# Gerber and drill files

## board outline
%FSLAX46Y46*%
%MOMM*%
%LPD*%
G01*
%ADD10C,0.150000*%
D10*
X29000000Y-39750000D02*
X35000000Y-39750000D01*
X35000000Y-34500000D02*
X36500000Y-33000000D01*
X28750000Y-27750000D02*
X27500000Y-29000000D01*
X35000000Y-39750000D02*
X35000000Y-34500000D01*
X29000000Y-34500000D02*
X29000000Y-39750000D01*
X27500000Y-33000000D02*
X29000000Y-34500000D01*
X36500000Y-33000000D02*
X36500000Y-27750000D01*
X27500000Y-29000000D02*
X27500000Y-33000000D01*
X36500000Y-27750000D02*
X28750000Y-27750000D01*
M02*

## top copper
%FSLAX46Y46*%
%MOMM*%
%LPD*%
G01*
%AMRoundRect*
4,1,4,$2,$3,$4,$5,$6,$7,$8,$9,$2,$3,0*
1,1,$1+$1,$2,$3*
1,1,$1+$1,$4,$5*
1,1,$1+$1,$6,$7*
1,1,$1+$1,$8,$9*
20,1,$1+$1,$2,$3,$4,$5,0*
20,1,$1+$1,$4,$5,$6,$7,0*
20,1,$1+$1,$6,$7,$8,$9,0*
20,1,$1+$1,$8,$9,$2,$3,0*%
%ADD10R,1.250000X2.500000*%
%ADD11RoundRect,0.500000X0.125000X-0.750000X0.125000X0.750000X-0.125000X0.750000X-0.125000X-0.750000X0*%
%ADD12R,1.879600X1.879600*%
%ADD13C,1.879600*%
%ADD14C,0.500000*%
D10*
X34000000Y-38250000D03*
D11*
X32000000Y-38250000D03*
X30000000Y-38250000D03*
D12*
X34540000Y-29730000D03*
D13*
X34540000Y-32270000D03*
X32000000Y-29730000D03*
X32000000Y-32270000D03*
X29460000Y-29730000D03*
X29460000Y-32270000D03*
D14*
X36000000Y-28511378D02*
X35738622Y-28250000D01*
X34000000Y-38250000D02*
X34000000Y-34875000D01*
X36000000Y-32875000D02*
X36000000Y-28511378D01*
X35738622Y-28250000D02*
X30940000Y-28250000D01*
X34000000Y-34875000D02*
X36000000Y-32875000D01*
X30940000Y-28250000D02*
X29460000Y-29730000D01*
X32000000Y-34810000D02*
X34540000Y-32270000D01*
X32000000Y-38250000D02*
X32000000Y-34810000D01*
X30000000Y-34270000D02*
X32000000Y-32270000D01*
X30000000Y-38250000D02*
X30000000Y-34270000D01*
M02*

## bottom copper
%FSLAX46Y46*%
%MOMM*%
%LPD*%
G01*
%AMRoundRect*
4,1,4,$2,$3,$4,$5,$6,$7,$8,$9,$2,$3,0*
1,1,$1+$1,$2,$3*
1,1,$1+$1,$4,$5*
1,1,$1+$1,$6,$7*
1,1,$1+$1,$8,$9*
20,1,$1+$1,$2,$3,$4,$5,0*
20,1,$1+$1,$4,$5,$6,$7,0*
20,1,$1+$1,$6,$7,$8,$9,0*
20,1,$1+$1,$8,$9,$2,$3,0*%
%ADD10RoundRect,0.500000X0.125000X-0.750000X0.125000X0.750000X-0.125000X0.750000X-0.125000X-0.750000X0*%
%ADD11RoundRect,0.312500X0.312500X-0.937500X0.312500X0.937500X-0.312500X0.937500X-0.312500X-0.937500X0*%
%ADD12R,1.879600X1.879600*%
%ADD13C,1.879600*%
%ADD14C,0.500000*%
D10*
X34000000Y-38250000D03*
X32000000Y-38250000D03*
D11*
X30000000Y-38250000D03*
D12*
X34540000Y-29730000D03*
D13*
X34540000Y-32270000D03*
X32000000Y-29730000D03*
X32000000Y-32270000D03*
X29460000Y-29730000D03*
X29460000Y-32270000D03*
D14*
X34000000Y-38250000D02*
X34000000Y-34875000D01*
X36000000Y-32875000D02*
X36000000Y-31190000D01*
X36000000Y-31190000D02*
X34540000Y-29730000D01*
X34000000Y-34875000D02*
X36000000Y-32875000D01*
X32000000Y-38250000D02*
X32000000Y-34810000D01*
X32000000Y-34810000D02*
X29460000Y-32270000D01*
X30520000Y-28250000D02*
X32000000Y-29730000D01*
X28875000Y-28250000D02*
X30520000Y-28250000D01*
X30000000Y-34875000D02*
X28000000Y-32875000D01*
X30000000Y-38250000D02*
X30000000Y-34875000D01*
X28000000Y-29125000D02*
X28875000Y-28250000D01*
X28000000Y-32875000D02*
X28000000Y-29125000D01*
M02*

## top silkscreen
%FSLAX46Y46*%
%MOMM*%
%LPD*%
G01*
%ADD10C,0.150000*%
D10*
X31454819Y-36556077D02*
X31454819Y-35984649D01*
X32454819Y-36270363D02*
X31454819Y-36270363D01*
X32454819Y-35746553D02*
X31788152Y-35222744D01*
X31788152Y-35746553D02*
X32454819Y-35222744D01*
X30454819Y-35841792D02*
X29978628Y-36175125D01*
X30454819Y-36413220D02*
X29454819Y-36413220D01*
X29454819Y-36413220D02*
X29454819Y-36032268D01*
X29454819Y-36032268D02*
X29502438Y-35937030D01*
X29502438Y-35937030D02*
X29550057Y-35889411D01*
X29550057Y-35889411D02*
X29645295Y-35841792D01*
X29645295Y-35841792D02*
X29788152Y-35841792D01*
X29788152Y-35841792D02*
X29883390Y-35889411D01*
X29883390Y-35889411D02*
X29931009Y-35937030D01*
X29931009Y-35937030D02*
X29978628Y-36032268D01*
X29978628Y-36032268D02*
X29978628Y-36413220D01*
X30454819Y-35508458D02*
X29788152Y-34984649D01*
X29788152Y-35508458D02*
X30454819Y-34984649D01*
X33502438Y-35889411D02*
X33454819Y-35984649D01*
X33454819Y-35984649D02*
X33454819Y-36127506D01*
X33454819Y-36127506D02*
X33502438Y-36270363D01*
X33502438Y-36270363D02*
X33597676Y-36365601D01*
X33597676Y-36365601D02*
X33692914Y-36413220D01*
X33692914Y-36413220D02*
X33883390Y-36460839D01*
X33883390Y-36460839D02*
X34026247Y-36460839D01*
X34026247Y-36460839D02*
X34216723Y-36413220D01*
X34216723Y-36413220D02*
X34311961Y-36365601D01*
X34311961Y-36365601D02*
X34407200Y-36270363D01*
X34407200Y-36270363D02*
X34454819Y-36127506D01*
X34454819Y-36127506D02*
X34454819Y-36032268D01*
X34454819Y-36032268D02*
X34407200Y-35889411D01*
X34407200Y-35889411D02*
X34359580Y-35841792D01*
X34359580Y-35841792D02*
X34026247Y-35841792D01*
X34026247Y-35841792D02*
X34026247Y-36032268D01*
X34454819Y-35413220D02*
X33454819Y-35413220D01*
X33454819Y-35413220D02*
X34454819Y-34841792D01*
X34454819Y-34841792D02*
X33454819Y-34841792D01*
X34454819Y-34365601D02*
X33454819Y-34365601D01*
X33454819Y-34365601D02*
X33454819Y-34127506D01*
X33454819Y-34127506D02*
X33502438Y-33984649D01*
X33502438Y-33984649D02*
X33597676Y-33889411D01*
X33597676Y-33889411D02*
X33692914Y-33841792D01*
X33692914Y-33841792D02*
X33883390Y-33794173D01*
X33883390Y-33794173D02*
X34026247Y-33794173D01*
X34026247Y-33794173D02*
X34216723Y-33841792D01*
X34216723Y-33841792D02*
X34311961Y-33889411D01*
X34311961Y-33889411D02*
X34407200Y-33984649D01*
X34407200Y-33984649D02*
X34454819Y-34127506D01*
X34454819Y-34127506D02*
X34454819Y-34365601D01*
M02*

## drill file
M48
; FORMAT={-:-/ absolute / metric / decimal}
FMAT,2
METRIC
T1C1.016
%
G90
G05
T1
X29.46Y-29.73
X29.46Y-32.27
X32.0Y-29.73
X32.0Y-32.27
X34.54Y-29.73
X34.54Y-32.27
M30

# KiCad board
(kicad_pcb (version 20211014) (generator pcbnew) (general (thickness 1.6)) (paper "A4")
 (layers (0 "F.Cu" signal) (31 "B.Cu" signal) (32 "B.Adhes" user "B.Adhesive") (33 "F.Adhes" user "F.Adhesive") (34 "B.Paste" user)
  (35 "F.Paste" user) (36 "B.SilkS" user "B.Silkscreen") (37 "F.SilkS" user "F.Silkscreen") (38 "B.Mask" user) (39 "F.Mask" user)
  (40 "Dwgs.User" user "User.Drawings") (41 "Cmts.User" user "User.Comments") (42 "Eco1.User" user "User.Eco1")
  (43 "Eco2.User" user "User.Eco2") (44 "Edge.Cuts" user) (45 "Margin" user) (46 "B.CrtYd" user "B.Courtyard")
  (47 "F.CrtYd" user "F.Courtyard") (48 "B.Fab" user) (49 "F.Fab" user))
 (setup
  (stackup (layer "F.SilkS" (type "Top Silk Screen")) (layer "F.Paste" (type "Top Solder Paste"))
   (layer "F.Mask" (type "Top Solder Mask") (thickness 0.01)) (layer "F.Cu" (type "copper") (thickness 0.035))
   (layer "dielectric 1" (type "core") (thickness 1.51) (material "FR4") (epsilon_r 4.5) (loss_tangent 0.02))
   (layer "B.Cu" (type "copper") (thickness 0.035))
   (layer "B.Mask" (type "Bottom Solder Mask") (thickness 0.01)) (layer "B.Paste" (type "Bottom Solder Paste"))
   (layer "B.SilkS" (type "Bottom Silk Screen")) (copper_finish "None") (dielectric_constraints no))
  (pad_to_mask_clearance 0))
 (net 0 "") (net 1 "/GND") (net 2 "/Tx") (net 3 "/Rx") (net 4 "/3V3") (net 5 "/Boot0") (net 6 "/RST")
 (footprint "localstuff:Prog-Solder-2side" (layer "F.Cu") (at 32 38.25 90)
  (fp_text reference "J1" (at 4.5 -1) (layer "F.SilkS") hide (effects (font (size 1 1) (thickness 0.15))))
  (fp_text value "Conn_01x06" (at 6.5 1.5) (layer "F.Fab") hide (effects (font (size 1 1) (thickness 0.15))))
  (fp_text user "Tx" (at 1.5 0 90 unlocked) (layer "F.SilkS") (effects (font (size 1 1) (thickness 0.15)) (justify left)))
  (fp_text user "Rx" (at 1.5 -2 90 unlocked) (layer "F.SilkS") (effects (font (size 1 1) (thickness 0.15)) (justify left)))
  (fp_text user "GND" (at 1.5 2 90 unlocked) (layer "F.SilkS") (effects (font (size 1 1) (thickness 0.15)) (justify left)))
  (pad "1" smd rect (at 0 2 90) (size 2.5 1.25) (layers "F.Cu" "F.Mask") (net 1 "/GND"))
  (pad "2" smd roundrect (at 0 0 90) (size 2.5 1.25) (layers "F.Cu" "F.Mask") (roundrect_rratio 0.4) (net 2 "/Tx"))
  (pad "3" smd roundrect (at 0 -2 90) (size 2.5 1.25) (layers "F.Cu" "F.Mask") (roundrect_rratio 0.4) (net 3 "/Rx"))
  (pad "4" smd roundrect (at 0 2 90) (size 2.5 1.25) (layers "B.Cu" "B.Mask") (roundrect_rratio 0.4) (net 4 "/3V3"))
  (pad "5" smd roundrect (at 0 0 90) (size 2.5 1.25) (layers "B.Cu" "B.Mask") (roundrect_rratio 0.4) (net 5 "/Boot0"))
  (pad "6" smd roundrect (at 0 -2 90) (size 2.5 1.25) (layers "B.Cu" "B.Mask") (roundrect_rratio 0.25) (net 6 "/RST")))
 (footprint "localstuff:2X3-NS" (layer "F.Cu") (at 32 31 180)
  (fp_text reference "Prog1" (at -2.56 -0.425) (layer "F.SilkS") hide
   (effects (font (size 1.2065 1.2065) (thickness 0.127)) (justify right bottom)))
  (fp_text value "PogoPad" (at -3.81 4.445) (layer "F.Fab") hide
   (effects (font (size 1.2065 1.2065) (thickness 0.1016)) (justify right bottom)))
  (pad "1" thru_hole rect locked (at -2.54 1.27 180) (size 1.8796 1.8796) (drill 1.016) (layers *.Cu *.Mask) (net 4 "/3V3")
   (solder_mask_margin 0.1016))
  (pad "2" thru_hole circle locked (at -2.54 -1.27 180) (size 1.8796 1.8796) (drill 1.016) (layers *.Cu *.Mask) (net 2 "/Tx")
   (solder_mask_margin 0.1016))
  (pad "3" thru_hole circle locked (at 0 1.27 180) (size 1.8796 1.8796) (drill 1.016) (layers *.Cu *.Mask) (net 6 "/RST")
   (solder_mask_margin 0.1016))
  (pad "4" thru_hole circle locked (at 0 -1.27 180) (size 1.8796 1.8796) (drill 1.016) (layers *.Cu *.Mask) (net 3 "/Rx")
   (solder_mask_margin 0.1016))
  (pad "5" thru_hole circle locked (at 2.54 1.27 180) (size 1.8796 1.8796) (drill 1.016) (layers *.Cu *.Mask) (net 1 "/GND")
   (solder_mask_margin 0.1016))
  (pad "6" thru_hole circle locked (at 2.54 -1.27 180) (size 1.8796 1.8796) (drill 1.016) (layers *.Cu *.Mask) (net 5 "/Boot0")
   (solder_mask_margin 0.1016)))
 (gr_line (start 29 39.75) (end 35 39.75) (layer "Edge.Cuts") (width 0.15))
 (gr_line (start 35 34.5) (end 36.5 33) (layer "Edge.Cuts") (width 0.15))
 (gr_line (start 28.75 27.75) (end 27.5 29) (layer "Edge.Cuts") (width 0.15))
 (gr_line (start 35 39.75) (end 35 34.5) (layer "Edge.Cuts") (width 0.15))
 (gr_line (start 29 34.5) (end 29 39.75) (layer "Edge.Cuts") (width 0.15))
 (gr_line (start 27.5 33) (end 29 34.5) (layer "Edge.Cuts") (width 0.15))
 (gr_line (start 36.5 33) (end 36.5 27.75) (layer "Edge.Cuts") (width 0.15))
 (gr_line (start 27.5 29) (end 27.5 33) (layer "Edge.Cuts") (width 0.15))
 (gr_line (start 36.5 27.75) (end 28.75 27.75) (layer "Edge.Cuts") (width 0.15))
 (segment (start 36 28.511378) (end 35.738622 28.25) (width 0.5) (layer "F.Cu") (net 1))
 (segment (start 34 38.25) (end 34 34.875) (width 0.5) (layer "F.Cu") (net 1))
 (segment (start 36 32.875) (end 36 28.511378) (width 0.5) (layer "F.Cu") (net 1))
 (segment (start 35.738622 28.25) (end 30.94 28.25) (width 0.5) (layer "F.Cu") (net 1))
 (segment (start 34 34.875) (end 36 32.875) (width 0.5) (layer "F.Cu") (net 1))
 (segment (start 30.94 28.25) (end 29.46 29.73) (width 0.5) (layer "F.Cu") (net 1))
 (segment (start 32 34.81) (end 34.54 32.27) (width 0.5) (layer "F.Cu") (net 2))
 (segment (start 32 38.25) (end 32 34.81) (width 0.5) (layer "F.Cu") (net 2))
 (segment (start 30 34.27) (end 32 32.27) (width 0.5) (layer "F.Cu") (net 3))
 (segment (start 30 38.25) (end 30 34.27) (width 0.5) (layer "F.Cu") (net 3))
 (segment (start 34 38.25) (end 34 34.875) (width 0.5) (layer "B.Cu") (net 4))
 (segment (start 36 32.875) (end 36 31.19) (width 0.5) (layer "B.Cu") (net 4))
 (segment (start 36 31.19) (end 34.54 29.73) (width 0.5) (layer "B.Cu") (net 4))
 (segment (start 34 34.875) (end 36 32.875) (width 0.5) (layer "B.Cu") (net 4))
 (segment (start 32 38.25) (end 32 34.81) (width 0.5) (layer "B.Cu") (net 5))
 (segment (start 32 34.81) (end 29.46 32.27) (width 0.5) (layer "B.Cu") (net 5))
 (segment (start 30.52 28.25) (end 32 29.73) (width 0.5) (layer "B.Cu") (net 6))
 (segment (start 28.875 28.25) (end 30.52 28.25) (width 0.5) (layer "B.Cu") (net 6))
 (segment (start 30 34.875) (end 28 32.875) (width 0.5) (layer "B.Cu") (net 6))
 (segment (start 30 38.25) (end 30 34.875) (width 0.5) (layer "B.Cu") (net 6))
 (segment (start 28 29.125) (end 28.875 28.25) (width 0.5) (layer "B.Cu") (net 6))
 (segment (start 28 32.875) (end 28 29.125) (width 0.5) (layer "B.Cu") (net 6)))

